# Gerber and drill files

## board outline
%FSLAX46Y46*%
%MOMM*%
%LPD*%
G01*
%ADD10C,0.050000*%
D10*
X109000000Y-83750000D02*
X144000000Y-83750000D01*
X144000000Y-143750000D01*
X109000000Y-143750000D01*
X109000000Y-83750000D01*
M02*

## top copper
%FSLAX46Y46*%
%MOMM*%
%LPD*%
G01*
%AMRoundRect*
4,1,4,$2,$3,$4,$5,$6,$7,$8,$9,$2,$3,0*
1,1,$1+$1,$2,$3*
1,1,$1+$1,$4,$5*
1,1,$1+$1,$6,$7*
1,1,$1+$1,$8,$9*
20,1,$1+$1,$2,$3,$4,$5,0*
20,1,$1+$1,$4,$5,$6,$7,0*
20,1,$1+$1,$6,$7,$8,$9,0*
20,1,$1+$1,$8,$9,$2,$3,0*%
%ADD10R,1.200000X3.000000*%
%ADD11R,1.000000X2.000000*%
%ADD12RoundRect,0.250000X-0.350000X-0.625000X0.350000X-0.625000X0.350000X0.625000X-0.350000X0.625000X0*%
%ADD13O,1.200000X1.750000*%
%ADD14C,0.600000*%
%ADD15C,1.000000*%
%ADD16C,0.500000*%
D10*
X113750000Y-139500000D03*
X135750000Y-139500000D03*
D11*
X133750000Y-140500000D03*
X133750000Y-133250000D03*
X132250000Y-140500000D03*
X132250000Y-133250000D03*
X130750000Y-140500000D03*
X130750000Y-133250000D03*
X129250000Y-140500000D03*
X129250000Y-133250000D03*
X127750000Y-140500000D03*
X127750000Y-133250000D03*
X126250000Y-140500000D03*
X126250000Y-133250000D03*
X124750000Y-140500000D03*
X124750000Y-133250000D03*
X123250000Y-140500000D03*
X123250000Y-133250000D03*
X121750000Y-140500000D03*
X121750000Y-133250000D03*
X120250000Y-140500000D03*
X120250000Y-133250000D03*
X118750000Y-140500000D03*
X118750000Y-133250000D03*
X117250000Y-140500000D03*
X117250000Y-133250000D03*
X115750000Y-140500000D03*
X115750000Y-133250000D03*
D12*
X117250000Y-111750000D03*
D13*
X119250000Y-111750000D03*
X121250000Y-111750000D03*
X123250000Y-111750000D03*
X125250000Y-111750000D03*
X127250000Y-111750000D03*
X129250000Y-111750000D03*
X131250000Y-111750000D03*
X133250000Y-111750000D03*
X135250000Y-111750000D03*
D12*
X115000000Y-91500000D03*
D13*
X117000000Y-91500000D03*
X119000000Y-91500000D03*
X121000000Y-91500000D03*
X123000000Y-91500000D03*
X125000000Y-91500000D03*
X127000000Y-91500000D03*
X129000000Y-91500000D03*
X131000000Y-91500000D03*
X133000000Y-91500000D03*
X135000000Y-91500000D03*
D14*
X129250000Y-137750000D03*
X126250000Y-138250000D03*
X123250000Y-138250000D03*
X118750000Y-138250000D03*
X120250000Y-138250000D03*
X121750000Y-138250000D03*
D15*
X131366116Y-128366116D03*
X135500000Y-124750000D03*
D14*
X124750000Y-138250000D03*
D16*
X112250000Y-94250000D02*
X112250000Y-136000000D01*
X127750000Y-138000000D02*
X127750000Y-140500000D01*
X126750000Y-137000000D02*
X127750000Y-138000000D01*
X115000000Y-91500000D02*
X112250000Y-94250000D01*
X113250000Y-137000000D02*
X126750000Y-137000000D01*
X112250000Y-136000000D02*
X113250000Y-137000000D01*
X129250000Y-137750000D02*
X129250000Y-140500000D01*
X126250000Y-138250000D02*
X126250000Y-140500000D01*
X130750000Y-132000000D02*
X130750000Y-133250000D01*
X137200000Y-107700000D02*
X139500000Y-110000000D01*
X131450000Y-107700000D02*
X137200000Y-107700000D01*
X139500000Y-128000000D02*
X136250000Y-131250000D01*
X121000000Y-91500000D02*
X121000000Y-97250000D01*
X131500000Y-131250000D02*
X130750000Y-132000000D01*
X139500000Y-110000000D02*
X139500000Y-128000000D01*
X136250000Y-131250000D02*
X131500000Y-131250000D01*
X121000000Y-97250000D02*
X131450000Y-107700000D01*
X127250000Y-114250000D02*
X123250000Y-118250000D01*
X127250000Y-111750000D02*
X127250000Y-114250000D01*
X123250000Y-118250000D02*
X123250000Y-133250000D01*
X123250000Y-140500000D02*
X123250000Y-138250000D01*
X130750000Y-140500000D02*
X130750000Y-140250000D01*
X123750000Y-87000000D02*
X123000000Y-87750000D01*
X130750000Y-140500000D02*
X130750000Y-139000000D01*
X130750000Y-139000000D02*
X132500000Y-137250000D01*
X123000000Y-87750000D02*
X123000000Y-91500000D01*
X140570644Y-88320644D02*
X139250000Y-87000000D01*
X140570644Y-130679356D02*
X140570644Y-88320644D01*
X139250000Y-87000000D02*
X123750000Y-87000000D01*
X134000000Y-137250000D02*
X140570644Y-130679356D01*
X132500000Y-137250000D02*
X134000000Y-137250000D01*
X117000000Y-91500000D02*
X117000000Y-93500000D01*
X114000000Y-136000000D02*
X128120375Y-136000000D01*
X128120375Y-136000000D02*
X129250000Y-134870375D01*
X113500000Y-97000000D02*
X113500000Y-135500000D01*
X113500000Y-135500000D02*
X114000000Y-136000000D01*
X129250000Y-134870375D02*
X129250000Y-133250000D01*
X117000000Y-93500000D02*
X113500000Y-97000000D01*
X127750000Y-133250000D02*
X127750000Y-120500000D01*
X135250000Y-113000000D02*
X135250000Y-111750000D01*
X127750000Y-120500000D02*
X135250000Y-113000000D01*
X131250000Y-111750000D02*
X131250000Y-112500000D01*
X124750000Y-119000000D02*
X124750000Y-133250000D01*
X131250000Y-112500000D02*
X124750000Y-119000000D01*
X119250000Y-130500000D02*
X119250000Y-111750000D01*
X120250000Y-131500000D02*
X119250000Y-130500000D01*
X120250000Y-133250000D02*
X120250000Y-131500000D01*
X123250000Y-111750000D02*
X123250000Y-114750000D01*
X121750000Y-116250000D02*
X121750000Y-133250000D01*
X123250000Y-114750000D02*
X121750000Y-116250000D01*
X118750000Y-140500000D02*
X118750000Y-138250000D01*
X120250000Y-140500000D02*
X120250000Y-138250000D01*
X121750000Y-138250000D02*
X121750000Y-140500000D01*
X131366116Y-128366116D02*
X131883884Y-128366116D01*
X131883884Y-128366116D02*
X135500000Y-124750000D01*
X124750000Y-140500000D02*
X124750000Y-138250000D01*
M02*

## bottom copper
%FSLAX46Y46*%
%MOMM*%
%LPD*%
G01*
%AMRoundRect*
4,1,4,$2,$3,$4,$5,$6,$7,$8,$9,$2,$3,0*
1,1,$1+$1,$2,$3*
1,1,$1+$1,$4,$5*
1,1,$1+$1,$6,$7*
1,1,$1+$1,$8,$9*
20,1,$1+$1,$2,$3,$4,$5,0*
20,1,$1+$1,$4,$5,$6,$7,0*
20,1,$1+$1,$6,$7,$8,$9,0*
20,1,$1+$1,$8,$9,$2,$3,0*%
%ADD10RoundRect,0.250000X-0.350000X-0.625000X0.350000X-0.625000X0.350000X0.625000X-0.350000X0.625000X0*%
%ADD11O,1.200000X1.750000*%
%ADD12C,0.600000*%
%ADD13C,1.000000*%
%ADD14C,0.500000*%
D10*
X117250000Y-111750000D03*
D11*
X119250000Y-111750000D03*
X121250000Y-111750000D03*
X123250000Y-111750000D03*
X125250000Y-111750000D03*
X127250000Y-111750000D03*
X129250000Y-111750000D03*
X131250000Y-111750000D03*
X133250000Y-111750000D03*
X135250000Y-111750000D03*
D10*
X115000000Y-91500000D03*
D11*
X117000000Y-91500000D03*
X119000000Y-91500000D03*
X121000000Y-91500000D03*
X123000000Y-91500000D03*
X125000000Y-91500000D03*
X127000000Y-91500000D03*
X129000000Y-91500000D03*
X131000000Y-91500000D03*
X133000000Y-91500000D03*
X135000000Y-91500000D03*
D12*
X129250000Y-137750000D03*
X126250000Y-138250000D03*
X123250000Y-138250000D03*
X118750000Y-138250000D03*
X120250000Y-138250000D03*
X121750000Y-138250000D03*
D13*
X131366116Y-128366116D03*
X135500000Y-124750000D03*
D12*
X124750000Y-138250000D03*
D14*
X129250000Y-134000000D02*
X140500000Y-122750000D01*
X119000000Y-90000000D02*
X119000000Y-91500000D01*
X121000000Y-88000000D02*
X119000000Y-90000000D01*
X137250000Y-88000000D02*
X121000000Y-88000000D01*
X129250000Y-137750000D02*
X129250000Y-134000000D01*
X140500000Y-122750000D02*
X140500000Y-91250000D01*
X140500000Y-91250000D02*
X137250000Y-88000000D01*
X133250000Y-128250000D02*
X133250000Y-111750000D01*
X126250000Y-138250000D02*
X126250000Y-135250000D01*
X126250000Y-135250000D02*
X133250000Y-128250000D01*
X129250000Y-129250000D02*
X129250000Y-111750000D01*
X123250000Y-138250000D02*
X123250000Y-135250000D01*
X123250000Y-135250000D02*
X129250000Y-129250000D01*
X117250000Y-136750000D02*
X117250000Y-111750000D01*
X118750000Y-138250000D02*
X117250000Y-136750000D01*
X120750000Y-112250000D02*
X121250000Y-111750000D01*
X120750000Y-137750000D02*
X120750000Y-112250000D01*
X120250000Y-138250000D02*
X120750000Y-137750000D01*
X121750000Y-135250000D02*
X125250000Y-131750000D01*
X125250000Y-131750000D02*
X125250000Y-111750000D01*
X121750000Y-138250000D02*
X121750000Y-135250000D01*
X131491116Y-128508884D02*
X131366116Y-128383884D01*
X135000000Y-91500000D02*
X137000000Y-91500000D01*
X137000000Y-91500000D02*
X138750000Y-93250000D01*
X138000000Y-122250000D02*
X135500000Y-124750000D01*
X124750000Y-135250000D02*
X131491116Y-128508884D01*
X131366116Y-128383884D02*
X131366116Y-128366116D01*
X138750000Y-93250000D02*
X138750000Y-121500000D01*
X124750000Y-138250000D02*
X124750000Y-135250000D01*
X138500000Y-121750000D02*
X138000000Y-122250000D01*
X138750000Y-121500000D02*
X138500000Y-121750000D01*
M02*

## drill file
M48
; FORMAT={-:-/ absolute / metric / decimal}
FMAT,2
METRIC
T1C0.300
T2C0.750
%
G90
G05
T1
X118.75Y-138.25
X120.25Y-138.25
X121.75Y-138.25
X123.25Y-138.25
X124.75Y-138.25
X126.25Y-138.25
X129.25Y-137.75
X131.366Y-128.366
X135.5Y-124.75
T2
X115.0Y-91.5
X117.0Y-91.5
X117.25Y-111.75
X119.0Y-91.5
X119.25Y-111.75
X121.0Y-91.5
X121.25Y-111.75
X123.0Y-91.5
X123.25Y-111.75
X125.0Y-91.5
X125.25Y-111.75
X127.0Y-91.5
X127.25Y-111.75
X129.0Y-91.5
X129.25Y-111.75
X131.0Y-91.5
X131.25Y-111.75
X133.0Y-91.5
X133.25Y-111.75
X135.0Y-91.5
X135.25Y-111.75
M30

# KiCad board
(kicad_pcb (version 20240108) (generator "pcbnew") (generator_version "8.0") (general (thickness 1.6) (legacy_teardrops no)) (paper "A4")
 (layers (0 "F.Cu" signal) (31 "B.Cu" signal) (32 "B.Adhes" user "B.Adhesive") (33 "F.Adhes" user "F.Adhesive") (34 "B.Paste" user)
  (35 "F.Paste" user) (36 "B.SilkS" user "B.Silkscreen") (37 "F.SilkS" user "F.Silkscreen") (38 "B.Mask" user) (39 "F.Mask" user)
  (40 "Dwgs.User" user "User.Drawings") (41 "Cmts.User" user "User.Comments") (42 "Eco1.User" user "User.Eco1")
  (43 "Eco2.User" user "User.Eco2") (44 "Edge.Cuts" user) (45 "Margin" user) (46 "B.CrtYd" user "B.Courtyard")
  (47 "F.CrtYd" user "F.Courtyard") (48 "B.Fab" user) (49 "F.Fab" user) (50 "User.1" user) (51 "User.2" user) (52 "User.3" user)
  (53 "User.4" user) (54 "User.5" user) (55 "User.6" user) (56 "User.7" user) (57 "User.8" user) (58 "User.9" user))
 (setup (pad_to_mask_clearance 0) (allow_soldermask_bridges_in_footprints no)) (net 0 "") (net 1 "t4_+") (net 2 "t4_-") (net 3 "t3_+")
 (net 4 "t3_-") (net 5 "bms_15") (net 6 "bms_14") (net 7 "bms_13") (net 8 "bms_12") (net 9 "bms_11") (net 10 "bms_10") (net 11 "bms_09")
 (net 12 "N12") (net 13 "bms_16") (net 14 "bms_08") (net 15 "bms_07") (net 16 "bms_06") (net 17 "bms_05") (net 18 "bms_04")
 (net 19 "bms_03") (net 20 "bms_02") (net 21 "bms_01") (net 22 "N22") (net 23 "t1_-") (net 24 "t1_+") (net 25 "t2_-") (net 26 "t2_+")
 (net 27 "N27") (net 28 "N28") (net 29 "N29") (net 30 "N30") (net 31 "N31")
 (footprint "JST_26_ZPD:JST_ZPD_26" (layer "F.Cu") (at 124.75 140.5)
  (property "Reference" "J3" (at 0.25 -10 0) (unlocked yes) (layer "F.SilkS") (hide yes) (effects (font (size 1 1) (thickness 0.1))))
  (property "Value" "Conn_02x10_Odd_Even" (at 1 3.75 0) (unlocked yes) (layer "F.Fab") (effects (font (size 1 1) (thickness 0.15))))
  (pad "" smd rect (at -10.5 -2.5) (size 1.2 3) (drill (offset -0.5 1.5)) (layers "F.Cu" "F.Paste" "F.Mask"))
  (pad "" smd rect (at 10.5 -2.5) (size 1.2 3) (drill (offset 0.5 1.5)) (layers "F.Cu" "F.Paste" "F.Mask"))
  (pad "1" smd rect (at 9 0) (size 1 2) (layers "F.Cu" "F.Paste" "F.Mask") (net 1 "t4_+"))
  (pad "2" smd rect (at 9 -7.25) (size 1 2) (layers "F.Cu" "F.Paste" "F.Mask") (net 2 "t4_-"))
  (pad "3" smd rect (at 7.5 0) (size 1 2) (layers "F.Cu" "F.Paste" "F.Mask") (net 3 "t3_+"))
  (pad "4" smd rect (at 7.5 -7.25) (size 1 2) (layers "F.Cu" "F.Paste" "F.Mask") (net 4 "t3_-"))
  (pad "5" smd rect (at 6 0) (size 1 2) (layers "F.Cu" "F.Paste" "F.Mask") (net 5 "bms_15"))
  (pad "6" smd rect (at 6 -7.25) (size 1 2) (layers "F.Cu" "F.Paste" "F.Mask") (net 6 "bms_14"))
  (pad "7" smd rect (at 4.5 0) (size 1 2) (layers "F.Cu" "F.Paste" "F.Mask") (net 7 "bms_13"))
  (pad "8" smd rect (at 4.5 -7.25) (size 1 2) (layers "F.Cu" "F.Paste" "F.Mask") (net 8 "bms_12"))
  (pad "9" smd rect (at 3 0) (size 1 2) (layers "F.Cu" "F.Paste" "F.Mask") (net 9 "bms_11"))
  (pad "10" smd rect (at 3 -7.25) (size 1 2) (layers "F.Cu" "F.Paste" "F.Mask") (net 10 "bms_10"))
  (pad "11" smd rect (at 1.5 0) (size 1 2) (layers "F.Cu" "F.Paste" "F.Mask") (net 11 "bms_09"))
  (pad "12" smd rect (at 1.5 -7.25) (size 1 2) (layers "F.Cu" "F.Paste" "F.Mask") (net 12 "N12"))
  (pad "13" smd rect (at 0 0) (size 1 2) (layers "F.Cu" "F.Paste" "F.Mask") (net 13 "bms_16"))
  (pad "14" smd rect (at 0 -7.25) (size 1 2) (layers "F.Cu" "F.Paste" "F.Mask") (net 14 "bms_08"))
  (pad "15" smd rect (at -1.5 0) (size 1 2) (layers "F.Cu" "F.Paste" "F.Mask") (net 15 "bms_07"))
  (pad "16" smd rect (at -1.5 -7.25) (size 1 2) (layers "F.Cu" "F.Paste" "F.Mask") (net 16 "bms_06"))
  (pad "17" smd rect (at -3 0) (size 1 2) (layers "F.Cu" "F.Paste" "F.Mask") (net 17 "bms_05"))
  (pad "18" smd rect (at -3 -7.25) (size 1 2) (layers "F.Cu" "F.Paste" "F.Mask") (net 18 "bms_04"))
  (pad "19" smd rect (at -4.5 0) (size 1 2) (layers "F.Cu" "F.Paste" "F.Mask") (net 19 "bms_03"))
  (pad "20" smd rect (at -4.5 -7.25) (size 1 2) (layers "F.Cu" "F.Paste" "F.Mask") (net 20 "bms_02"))
  (pad "21" smd rect (at -6 0) (size 1 2) (layers "F.Cu" "F.Paste" "F.Mask") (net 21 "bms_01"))
  (pad "22" smd rect (at -6 -7.25) (size 1 2) (layers "F.Cu" "F.Paste" "F.Mask") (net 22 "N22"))
  (pad "23" smd rect (at -7.5 0) (size 1 2) (layers "F.Cu" "F.Paste" "F.Mask") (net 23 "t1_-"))
  (pad "24" smd rect (at -7.5 -7.25) (size 1 2) (layers "F.Cu" "F.Paste" "F.Mask") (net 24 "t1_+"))
  (pad "25" smd rect (at -9 0) (size 1 2) (layers "F.Cu" "F.Paste" "F.Mask") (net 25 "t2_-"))
  (pad "26" smd rect (at -9 -7.25) (size 1 2) (layers "F.Cu" "F.Paste" "F.Mask") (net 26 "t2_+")))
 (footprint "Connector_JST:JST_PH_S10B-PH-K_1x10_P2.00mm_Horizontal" (layer "F.Cu") (at 117.25 111.75)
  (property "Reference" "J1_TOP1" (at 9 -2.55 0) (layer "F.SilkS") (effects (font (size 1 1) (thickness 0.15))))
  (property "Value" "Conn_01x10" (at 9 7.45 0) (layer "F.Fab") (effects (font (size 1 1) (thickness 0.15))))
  (pad "1" thru_hole roundrect (at 0 0) (size 1.2 1.75) (drill 0.75) (layers "*.Cu" "*.Mask") (remove_unused_layers no)
   (roundrect_rratio 0.208333) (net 21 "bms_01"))
  (pad "2" thru_hole oval (at 2 0) (size 1.2 1.75) (drill 0.75) (layers "*.Cu" "*.Mask") (remove_unused_layers no) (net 20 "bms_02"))
  (pad "3" thru_hole oval (at 4 0) (size 1.2 1.75) (drill 0.75) (layers "*.Cu" "*.Mask") (remove_unused_layers no) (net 19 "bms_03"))
  (pad "4" thru_hole oval (at 6 0) (size 1.2 1.75) (drill 0.75) (layers "*.Cu" "*.Mask") (remove_unused_layers no) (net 18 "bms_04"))
  (pad "5" thru_hole oval (at 8 0) (size 1.2 1.75) (drill 0.75) (layers "*.Cu" "*.Mask") (remove_unused_layers no) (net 17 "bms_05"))
  (pad "6" thru_hole oval (at 10 0) (size 1.2 1.75) (drill 0.75) (layers "*.Cu" "*.Mask") (remove_unused_layers no) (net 16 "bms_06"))
  (pad "7" thru_hole oval (at 12 0) (size 1.2 1.75) (drill 0.75) (layers "*.Cu" "*.Mask") (remove_unused_layers no) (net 15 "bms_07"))
  (pad "8" thru_hole oval (at 14 0) (size 1.2 1.75) (drill 0.75) (layers "*.Cu" "*.Mask") (remove_unused_layers no) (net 14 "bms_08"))
  (pad "9" thru_hole oval (at 16 0) (size 1.2 1.75) (drill 0.75) (layers "*.Cu" "*.Mask") (remove_unused_layers no) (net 11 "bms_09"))
  (pad "10" thru_hole oval (at 18 0) (size 1.2 1.75) (drill 0.75) (layers "*.Cu" "*.Mask") (remove_unused_layers no) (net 10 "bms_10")))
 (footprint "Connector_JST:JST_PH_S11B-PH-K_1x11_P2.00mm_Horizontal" (layer "F.Cu") (at 115 91.5)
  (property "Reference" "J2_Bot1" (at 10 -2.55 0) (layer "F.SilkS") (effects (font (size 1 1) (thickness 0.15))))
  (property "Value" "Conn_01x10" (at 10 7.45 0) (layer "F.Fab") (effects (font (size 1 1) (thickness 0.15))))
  (pad "1" thru_hole roundrect (at 0 0) (size 1.2 1.75) (drill 0.75) (layers "*.Cu" "*.Mask") (remove_unused_layers no)
   (roundrect_rratio 0.208333) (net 9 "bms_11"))
  (pad "2" thru_hole oval (at 2 0) (size 1.2 1.75) (drill 0.75) (layers "*.Cu" "*.Mask") (remove_unused_layers no) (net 8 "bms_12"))
  (pad "3" thru_hole oval (at 4 0) (size 1.2 1.75) (drill 0.75) (layers "*.Cu" "*.Mask") (remove_unused_layers no) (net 7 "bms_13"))
  (pad "4" thru_hole oval (at 6 0) (size 1.2 1.75) (drill 0.75) (layers "*.Cu" "*.Mask") (remove_unused_layers no) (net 6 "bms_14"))
  (pad "5" thru_hole oval (at 8 0) (size 1.2 1.75) (drill 0.75) (layers "*.Cu" "*.Mask") (remove_unused_layers no) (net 5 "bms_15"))
  (pad "6" thru_hole oval (at 10 0) (size 1.2 1.75) (drill 0.75) (layers "*.Cu" "*.Mask") (remove_unused_layers no) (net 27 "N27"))
  (pad "7" thru_hole oval (at 12 0) (size 1.2 1.75) (drill 0.75) (layers "*.Cu" "*.Mask") (remove_unused_layers no) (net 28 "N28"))
  (pad "8" thru_hole oval (at 14 0) (size 1.2 1.75) (drill 0.75) (layers "*.Cu" "*.Mask") (remove_unused_layers no) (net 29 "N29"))
  (pad "9" thru_hole oval (at 16 0) (size 1.2 1.75) (drill 0.75) (layers "*.Cu" "*.Mask") (remove_unused_layers no) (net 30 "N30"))
  (pad "10" thru_hole oval (at 18 0) (size 1.2 1.75) (drill 0.75) (layers "*.Cu" "*.Mask") (remove_unused_layers no) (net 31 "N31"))
  (pad "11" thru_hole oval (at 20 0) (size 1.2 1.75) (drill 0.75) (layers "*.Cu" "*.Mask") (remove_unused_layers no) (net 13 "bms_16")))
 (gr_rect (start 109 83.75) (end 144 143.75) (stroke (width 0.05) (type default)) (fill none) (layer "Edge.Cuts"))
 (segment (start 112.25 94.25) (end 112.25 136) (width 0.5) (layer "F.Cu") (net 9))
 (segment (start 127.75 138) (end 127.75 140.5) (width 0.5) (layer "F.Cu") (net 9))
 (segment (start 126.75 137) (end 127.75 138) (width 0.5) (layer "F.Cu") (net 9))
 (segment (start 115 91.5) (end 112.25 94.25) (width 0.5) (layer "F.Cu") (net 9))
 (segment (start 113.25 137) (end 126.75 137) (width 0.5) (layer "F.Cu") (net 9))
 (segment (start 112.25 136) (end 113.25 137) (width 0.5) (layer "F.Cu") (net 9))
 (segment (start 129.25 137.75) (end 129.25 140.5) (width 0.5) (layer "F.Cu") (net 7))
 (via (at 129.25 137.75) (size 0.6) (drill 0.3) (layers "F.Cu" "B.Cu") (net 7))
 (segment (start 129.25 134) (end 140.5 122.75) (width 0.5) (layer "B.Cu") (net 7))
 (segment (start 119 90) (end 119 91.5) (width 0.5) (layer "B.Cu") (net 7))
 (segment (start 121 88) (end 119 90) (width 0.5) (layer "B.Cu") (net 7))
 (segment (start 137.25 88) (end 121 88) (width 0.5) (layer "B.Cu") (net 7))
 (segment (start 129.25 137.75) (end 129.25 134) (width 0.5) (layer "B.Cu") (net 7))
 (segment (start 140.5 122.75) (end 140.5 91.25) (width 0.5) (layer "B.Cu") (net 7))
 (segment (start 140.5 91.25) (end 137.25 88) (width 0.5) (layer "B.Cu") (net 7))
 (segment (start 126.25 138.25) (end 126.25 140.5) (width 0.5) (layer "F.Cu") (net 11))
 (via (at 126.25 138.25) (size 0.6) (drill 0.3) (layers "F.Cu" "B.Cu") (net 11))
 (segment (start 133.25 128.25) (end 133.25 111.75) (width 0.5) (layer "B.Cu") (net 11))
 (segment (start 126.25 138.25) (end 126.25 135.25) (width 0.5) (layer "B.Cu") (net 11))
 (segment (start 126.25 135.25) (end 133.25 128.25) (width 0.5) (layer "B.Cu") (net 11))
 (segment (start 130.75 132) (end 130.75 133.25) (width 0.5) (layer "F.Cu") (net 6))
 (segment (start 137.2 107.7) (end 139.5 110) (width 0.5) (layer "F.Cu") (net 6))
 (segment (start 131.45 107.7) (end 137.2 107.7) (width 0.5) (layer "F.Cu") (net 6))
 (segment (start 139.5 128) (end 136.25 131.25) (width 0.5) (layer "F.Cu") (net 6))
 (segment (start 121 91.5) (end 121 97.25) (width 0.5) (layer "F.Cu") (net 6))
 (segment (start 131.5 131.25) (end 130.75 132) (width 0.5) (layer "F.Cu") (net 6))
 (segment (start 139.5 110) (end 139.5 128) (width 0.5) (layer "F.Cu") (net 6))
 (segment (start 136.25 131.25) (end 131.5 131.25) (width 0.5) (layer "F.Cu") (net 6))
 (segment (start 121 97.25) (end 131.45 107.7) (width 0.5) (layer "F.Cu") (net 6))
 (segment (start 127.25 114.25) (end 123.25 118.25) (width 0.5) (layer "F.Cu") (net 16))
 (segment (start 127.25 111.75) (end 127.25 114.25) (width 0.5) (layer "F.Cu") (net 16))
 (segment (start 123.25 118.25) (end 123.25 133.25) (width 0.5) (layer "F.Cu") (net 16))
 (segment (start 123.25 140.5) (end 123.25 138.25) (width 0.5) (layer "F.Cu") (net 15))
 (via (at 123.25 138.25) (size 0.6) (drill 0.3) (layers "F.Cu" "B.Cu") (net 15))
 (segment (start 129.25 129.25) (end 129.25 111.75) (width 0.5) (layer "B.Cu") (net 15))
 (segment (start 123.25 138.25) (end 123.25 135.25) (width 0.5) (layer "B.Cu") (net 15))
 (segment (start 123.25 135.25) (end 129.25 129.25) (width 0.5) (layer "B.Cu") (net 15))
 (segment (start 130.75 140.5) (end 130.75 140.25) (width 0.5) (layer "F.Cu") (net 5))
 (segment (start 123.75 87) (end 123 87.75) (width 0.5) (layer "F.Cu") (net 5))
 (segment (start 130.75 140.5) (end 130.75 139) (width 0.5) (layer "F.Cu") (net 5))
 (segment (start 130.75 139) (end 132.5 137.25) (width 0.5) (layer "F.Cu") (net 5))
 (segment (start 123 87.75) (end 123 91.5) (width 0.5) (layer "F.Cu") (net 5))
 (segment (start 140.570644 88.320644) (end 139.25 87) (width 0.5) (layer "F.Cu") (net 5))
 (segment (start 140.570644 130.679356) (end 140.570644 88.320644) (width 0.5) (layer "F.Cu") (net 5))
 (segment (start 139.25 87) (end 123.75 87) (width 0.5) (layer "F.Cu") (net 5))
 (segment (start 134 137.25) (end 140.570644 130.679356) (width 0.5) (layer "F.Cu") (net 5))
 (segment (start 132.5 137.25) (end 134 137.25) (width 0.5) (layer "F.Cu") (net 5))
 (segment (start 117 91.5) (end 117 93.5) (width 0.5) (layer "F.Cu") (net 8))
 (segment (start 114 136) (end 128.120375 136) (width 0.5) (layer "F.Cu") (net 8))
 (segment (start 128.120375 136) (end 129.25 134.870375) (width 0.5) (layer "F.Cu") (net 8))
 (segment (start 113.5 97) (end 113.5 135.5) (width 0.5) (layer "F.Cu") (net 8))
 (segment (start 113.5 135.5) (end 114 136) (width 0.5) (layer "F.Cu") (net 8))
 (segment (start 129.25 134.870375) (end 129.25 133.25) (width 0.5) (layer "F.Cu") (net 8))
 (segment (start 117 93.5) (end 113.5 97) (width 0.5) (layer "F.Cu") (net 8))
 (segment (start 127.75 133.25) (end 127.75 120.5) (width 0.5) (layer "F.Cu") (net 10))
 (segment (start 135.25 113) (end 135.25 111.75) (width 0.5) (layer "F.Cu") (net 10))
 (segment (start 127.75 120.5) (end 135.25 113) (width 0.5) (layer "F.Cu") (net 10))
 (segment (start 131.25 111.75) (end 131.25 112.5) (width 0.5) (layer "F.Cu") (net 14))
 (segment (start 124.75 119) (end 124.75 133.25) (width 0.5) (layer "F.Cu") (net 14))
 (segment (start 131.25 112.5) (end 124.75 119) (width 0.5) (layer "F.Cu") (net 14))
 (segment (start 119.25 130.5) (end 119.25 111.75) (width 0.5) (layer "F.Cu") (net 20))
 (segment (start 120.25 131.5) (end 119.25 130.5) (width 0.5) (layer "F.Cu") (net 20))
 (segment (start 120.25 133.25) (end 120.25 131.5) (width 0.5) (layer "F.Cu") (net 20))
 (segment (start 123.25 111.75) (end 123.25 114.75) (width 0.5) (layer "F.Cu") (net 18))
 (segment (start 121.75 116.25) (end 121.75 133.25) (width 0.5) (layer "F.Cu") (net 18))
 (segment (start 123.25 114.75) (end 121.75 116.25) (width 0.5) (layer "F.Cu") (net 18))
 (segment (start 118.75 140.5) (end 118.75 138.25) (width 0.5) (layer "F.Cu") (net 21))
 (via (at 118.75 138.25) (size 0.6) (drill 0.3) (layers "F.Cu" "B.Cu") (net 21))
 (segment (start 117.25 136.75) (end 117.25 111.75) (width 0.5) (layer "B.Cu") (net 21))
 (segment (start 118.75 138.25) (end 117.25 136.75) (width 0.5) (layer "B.Cu") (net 21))
 (segment (start 120.25 140.5) (end 120.25 138.25) (width 0.5) (layer "F.Cu") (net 19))
 (via (at 120.25 138.25) (size 0.6) (drill 0.3) (layers "F.Cu" "B.Cu") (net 19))
 (segment (start 120.75 112.25) (end 121.25 111.75) (width 0.5) (layer "B.Cu") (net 19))
 (segment (start 120.75 137.75) (end 120.75 112.25) (width 0.5) (layer "B.Cu") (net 19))
 (segment (start 120.25 138.25) (end 120.75 137.75) (width 0.5) (layer "B.Cu") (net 19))
 (segment (start 121.75 138.25) (end 121.75 140.5) (width 0.5) (layer "F.Cu") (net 17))
 (via (at 121.75 138.25) (size 0.6) (drill 0.3) (layers "F.Cu" "B.Cu") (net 17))
 (segment (start 121.75 135.25) (end 125.25 131.75) (width 0.5) (layer "B.Cu") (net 17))
 (segment (start 125.25 131.75) (end 125.25 111.75) (width 0.5) (layer "B.Cu") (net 17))
 (segment (start 121.75 138.25) (end 121.75 135.25) (width 0.5) (layer "B.Cu") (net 17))
 (segment (start 131.366116 128.366116) (end 131.883884 128.366116) (width 0.5) (layer "F.Cu") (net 13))
 (segment (start 131.883884 128.366116) (end 135.5 124.75) (width 0.5) (layer "F.Cu") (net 13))
 (segment (start 124.75 140.5) (end 124.75 138.25) (width 0.5) (layer "F.Cu") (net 13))
 (via (at 131.366116 128.366116) (size 1) (drill 0.3) (layers "F.Cu" "B.Cu") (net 13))
 (via (at 135.5 124.75) (size 1) (drill 0.3) (layers "F.Cu" "B.Cu") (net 13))
 (via (at 124.75 138.25) (size 0.6) (drill 0.3) (layers "F.Cu" "B.Cu") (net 13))
 (segment (start 131.491116 128.508884) (end 131.366116 128.383884) (width 0.5) (layer "B.Cu") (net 13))
 (segment (start 135 91.5) (end 137 91.5) (width 0.5) (layer "B.Cu") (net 13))
 (segment (start 137 91.5) (end 138.75 93.25) (width 0.5) (layer "B.Cu") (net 13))
 (segment (start 138 122.25) (end 135.5 124.75) (width 0.5) (layer "B.Cu") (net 13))
 (segment (start 124.75 135.25) (end 131.491116 128.508884) (width 0.5) (layer "B.Cu") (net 13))
 (segment (start 131.366116 128.383884) (end 131.366116 128.366116) (width 0.5) (layer "B.Cu") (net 13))
 (segment (start 138.75 93.25) (end 138.75 121.5) (width 0.5) (layer "B.Cu") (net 13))
 (segment (start 124.75 138.25) (end 124.75 135.25) (width 0.5) (layer "B.Cu") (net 13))
 (segment (start 138.5 121.75) (end 138 122.25) (width 0.5) (layer "B.Cu") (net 13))
 (segment (start 138.75 121.5) (end 138.5 121.75) (width 0.5) (layer "B.Cu") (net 13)))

